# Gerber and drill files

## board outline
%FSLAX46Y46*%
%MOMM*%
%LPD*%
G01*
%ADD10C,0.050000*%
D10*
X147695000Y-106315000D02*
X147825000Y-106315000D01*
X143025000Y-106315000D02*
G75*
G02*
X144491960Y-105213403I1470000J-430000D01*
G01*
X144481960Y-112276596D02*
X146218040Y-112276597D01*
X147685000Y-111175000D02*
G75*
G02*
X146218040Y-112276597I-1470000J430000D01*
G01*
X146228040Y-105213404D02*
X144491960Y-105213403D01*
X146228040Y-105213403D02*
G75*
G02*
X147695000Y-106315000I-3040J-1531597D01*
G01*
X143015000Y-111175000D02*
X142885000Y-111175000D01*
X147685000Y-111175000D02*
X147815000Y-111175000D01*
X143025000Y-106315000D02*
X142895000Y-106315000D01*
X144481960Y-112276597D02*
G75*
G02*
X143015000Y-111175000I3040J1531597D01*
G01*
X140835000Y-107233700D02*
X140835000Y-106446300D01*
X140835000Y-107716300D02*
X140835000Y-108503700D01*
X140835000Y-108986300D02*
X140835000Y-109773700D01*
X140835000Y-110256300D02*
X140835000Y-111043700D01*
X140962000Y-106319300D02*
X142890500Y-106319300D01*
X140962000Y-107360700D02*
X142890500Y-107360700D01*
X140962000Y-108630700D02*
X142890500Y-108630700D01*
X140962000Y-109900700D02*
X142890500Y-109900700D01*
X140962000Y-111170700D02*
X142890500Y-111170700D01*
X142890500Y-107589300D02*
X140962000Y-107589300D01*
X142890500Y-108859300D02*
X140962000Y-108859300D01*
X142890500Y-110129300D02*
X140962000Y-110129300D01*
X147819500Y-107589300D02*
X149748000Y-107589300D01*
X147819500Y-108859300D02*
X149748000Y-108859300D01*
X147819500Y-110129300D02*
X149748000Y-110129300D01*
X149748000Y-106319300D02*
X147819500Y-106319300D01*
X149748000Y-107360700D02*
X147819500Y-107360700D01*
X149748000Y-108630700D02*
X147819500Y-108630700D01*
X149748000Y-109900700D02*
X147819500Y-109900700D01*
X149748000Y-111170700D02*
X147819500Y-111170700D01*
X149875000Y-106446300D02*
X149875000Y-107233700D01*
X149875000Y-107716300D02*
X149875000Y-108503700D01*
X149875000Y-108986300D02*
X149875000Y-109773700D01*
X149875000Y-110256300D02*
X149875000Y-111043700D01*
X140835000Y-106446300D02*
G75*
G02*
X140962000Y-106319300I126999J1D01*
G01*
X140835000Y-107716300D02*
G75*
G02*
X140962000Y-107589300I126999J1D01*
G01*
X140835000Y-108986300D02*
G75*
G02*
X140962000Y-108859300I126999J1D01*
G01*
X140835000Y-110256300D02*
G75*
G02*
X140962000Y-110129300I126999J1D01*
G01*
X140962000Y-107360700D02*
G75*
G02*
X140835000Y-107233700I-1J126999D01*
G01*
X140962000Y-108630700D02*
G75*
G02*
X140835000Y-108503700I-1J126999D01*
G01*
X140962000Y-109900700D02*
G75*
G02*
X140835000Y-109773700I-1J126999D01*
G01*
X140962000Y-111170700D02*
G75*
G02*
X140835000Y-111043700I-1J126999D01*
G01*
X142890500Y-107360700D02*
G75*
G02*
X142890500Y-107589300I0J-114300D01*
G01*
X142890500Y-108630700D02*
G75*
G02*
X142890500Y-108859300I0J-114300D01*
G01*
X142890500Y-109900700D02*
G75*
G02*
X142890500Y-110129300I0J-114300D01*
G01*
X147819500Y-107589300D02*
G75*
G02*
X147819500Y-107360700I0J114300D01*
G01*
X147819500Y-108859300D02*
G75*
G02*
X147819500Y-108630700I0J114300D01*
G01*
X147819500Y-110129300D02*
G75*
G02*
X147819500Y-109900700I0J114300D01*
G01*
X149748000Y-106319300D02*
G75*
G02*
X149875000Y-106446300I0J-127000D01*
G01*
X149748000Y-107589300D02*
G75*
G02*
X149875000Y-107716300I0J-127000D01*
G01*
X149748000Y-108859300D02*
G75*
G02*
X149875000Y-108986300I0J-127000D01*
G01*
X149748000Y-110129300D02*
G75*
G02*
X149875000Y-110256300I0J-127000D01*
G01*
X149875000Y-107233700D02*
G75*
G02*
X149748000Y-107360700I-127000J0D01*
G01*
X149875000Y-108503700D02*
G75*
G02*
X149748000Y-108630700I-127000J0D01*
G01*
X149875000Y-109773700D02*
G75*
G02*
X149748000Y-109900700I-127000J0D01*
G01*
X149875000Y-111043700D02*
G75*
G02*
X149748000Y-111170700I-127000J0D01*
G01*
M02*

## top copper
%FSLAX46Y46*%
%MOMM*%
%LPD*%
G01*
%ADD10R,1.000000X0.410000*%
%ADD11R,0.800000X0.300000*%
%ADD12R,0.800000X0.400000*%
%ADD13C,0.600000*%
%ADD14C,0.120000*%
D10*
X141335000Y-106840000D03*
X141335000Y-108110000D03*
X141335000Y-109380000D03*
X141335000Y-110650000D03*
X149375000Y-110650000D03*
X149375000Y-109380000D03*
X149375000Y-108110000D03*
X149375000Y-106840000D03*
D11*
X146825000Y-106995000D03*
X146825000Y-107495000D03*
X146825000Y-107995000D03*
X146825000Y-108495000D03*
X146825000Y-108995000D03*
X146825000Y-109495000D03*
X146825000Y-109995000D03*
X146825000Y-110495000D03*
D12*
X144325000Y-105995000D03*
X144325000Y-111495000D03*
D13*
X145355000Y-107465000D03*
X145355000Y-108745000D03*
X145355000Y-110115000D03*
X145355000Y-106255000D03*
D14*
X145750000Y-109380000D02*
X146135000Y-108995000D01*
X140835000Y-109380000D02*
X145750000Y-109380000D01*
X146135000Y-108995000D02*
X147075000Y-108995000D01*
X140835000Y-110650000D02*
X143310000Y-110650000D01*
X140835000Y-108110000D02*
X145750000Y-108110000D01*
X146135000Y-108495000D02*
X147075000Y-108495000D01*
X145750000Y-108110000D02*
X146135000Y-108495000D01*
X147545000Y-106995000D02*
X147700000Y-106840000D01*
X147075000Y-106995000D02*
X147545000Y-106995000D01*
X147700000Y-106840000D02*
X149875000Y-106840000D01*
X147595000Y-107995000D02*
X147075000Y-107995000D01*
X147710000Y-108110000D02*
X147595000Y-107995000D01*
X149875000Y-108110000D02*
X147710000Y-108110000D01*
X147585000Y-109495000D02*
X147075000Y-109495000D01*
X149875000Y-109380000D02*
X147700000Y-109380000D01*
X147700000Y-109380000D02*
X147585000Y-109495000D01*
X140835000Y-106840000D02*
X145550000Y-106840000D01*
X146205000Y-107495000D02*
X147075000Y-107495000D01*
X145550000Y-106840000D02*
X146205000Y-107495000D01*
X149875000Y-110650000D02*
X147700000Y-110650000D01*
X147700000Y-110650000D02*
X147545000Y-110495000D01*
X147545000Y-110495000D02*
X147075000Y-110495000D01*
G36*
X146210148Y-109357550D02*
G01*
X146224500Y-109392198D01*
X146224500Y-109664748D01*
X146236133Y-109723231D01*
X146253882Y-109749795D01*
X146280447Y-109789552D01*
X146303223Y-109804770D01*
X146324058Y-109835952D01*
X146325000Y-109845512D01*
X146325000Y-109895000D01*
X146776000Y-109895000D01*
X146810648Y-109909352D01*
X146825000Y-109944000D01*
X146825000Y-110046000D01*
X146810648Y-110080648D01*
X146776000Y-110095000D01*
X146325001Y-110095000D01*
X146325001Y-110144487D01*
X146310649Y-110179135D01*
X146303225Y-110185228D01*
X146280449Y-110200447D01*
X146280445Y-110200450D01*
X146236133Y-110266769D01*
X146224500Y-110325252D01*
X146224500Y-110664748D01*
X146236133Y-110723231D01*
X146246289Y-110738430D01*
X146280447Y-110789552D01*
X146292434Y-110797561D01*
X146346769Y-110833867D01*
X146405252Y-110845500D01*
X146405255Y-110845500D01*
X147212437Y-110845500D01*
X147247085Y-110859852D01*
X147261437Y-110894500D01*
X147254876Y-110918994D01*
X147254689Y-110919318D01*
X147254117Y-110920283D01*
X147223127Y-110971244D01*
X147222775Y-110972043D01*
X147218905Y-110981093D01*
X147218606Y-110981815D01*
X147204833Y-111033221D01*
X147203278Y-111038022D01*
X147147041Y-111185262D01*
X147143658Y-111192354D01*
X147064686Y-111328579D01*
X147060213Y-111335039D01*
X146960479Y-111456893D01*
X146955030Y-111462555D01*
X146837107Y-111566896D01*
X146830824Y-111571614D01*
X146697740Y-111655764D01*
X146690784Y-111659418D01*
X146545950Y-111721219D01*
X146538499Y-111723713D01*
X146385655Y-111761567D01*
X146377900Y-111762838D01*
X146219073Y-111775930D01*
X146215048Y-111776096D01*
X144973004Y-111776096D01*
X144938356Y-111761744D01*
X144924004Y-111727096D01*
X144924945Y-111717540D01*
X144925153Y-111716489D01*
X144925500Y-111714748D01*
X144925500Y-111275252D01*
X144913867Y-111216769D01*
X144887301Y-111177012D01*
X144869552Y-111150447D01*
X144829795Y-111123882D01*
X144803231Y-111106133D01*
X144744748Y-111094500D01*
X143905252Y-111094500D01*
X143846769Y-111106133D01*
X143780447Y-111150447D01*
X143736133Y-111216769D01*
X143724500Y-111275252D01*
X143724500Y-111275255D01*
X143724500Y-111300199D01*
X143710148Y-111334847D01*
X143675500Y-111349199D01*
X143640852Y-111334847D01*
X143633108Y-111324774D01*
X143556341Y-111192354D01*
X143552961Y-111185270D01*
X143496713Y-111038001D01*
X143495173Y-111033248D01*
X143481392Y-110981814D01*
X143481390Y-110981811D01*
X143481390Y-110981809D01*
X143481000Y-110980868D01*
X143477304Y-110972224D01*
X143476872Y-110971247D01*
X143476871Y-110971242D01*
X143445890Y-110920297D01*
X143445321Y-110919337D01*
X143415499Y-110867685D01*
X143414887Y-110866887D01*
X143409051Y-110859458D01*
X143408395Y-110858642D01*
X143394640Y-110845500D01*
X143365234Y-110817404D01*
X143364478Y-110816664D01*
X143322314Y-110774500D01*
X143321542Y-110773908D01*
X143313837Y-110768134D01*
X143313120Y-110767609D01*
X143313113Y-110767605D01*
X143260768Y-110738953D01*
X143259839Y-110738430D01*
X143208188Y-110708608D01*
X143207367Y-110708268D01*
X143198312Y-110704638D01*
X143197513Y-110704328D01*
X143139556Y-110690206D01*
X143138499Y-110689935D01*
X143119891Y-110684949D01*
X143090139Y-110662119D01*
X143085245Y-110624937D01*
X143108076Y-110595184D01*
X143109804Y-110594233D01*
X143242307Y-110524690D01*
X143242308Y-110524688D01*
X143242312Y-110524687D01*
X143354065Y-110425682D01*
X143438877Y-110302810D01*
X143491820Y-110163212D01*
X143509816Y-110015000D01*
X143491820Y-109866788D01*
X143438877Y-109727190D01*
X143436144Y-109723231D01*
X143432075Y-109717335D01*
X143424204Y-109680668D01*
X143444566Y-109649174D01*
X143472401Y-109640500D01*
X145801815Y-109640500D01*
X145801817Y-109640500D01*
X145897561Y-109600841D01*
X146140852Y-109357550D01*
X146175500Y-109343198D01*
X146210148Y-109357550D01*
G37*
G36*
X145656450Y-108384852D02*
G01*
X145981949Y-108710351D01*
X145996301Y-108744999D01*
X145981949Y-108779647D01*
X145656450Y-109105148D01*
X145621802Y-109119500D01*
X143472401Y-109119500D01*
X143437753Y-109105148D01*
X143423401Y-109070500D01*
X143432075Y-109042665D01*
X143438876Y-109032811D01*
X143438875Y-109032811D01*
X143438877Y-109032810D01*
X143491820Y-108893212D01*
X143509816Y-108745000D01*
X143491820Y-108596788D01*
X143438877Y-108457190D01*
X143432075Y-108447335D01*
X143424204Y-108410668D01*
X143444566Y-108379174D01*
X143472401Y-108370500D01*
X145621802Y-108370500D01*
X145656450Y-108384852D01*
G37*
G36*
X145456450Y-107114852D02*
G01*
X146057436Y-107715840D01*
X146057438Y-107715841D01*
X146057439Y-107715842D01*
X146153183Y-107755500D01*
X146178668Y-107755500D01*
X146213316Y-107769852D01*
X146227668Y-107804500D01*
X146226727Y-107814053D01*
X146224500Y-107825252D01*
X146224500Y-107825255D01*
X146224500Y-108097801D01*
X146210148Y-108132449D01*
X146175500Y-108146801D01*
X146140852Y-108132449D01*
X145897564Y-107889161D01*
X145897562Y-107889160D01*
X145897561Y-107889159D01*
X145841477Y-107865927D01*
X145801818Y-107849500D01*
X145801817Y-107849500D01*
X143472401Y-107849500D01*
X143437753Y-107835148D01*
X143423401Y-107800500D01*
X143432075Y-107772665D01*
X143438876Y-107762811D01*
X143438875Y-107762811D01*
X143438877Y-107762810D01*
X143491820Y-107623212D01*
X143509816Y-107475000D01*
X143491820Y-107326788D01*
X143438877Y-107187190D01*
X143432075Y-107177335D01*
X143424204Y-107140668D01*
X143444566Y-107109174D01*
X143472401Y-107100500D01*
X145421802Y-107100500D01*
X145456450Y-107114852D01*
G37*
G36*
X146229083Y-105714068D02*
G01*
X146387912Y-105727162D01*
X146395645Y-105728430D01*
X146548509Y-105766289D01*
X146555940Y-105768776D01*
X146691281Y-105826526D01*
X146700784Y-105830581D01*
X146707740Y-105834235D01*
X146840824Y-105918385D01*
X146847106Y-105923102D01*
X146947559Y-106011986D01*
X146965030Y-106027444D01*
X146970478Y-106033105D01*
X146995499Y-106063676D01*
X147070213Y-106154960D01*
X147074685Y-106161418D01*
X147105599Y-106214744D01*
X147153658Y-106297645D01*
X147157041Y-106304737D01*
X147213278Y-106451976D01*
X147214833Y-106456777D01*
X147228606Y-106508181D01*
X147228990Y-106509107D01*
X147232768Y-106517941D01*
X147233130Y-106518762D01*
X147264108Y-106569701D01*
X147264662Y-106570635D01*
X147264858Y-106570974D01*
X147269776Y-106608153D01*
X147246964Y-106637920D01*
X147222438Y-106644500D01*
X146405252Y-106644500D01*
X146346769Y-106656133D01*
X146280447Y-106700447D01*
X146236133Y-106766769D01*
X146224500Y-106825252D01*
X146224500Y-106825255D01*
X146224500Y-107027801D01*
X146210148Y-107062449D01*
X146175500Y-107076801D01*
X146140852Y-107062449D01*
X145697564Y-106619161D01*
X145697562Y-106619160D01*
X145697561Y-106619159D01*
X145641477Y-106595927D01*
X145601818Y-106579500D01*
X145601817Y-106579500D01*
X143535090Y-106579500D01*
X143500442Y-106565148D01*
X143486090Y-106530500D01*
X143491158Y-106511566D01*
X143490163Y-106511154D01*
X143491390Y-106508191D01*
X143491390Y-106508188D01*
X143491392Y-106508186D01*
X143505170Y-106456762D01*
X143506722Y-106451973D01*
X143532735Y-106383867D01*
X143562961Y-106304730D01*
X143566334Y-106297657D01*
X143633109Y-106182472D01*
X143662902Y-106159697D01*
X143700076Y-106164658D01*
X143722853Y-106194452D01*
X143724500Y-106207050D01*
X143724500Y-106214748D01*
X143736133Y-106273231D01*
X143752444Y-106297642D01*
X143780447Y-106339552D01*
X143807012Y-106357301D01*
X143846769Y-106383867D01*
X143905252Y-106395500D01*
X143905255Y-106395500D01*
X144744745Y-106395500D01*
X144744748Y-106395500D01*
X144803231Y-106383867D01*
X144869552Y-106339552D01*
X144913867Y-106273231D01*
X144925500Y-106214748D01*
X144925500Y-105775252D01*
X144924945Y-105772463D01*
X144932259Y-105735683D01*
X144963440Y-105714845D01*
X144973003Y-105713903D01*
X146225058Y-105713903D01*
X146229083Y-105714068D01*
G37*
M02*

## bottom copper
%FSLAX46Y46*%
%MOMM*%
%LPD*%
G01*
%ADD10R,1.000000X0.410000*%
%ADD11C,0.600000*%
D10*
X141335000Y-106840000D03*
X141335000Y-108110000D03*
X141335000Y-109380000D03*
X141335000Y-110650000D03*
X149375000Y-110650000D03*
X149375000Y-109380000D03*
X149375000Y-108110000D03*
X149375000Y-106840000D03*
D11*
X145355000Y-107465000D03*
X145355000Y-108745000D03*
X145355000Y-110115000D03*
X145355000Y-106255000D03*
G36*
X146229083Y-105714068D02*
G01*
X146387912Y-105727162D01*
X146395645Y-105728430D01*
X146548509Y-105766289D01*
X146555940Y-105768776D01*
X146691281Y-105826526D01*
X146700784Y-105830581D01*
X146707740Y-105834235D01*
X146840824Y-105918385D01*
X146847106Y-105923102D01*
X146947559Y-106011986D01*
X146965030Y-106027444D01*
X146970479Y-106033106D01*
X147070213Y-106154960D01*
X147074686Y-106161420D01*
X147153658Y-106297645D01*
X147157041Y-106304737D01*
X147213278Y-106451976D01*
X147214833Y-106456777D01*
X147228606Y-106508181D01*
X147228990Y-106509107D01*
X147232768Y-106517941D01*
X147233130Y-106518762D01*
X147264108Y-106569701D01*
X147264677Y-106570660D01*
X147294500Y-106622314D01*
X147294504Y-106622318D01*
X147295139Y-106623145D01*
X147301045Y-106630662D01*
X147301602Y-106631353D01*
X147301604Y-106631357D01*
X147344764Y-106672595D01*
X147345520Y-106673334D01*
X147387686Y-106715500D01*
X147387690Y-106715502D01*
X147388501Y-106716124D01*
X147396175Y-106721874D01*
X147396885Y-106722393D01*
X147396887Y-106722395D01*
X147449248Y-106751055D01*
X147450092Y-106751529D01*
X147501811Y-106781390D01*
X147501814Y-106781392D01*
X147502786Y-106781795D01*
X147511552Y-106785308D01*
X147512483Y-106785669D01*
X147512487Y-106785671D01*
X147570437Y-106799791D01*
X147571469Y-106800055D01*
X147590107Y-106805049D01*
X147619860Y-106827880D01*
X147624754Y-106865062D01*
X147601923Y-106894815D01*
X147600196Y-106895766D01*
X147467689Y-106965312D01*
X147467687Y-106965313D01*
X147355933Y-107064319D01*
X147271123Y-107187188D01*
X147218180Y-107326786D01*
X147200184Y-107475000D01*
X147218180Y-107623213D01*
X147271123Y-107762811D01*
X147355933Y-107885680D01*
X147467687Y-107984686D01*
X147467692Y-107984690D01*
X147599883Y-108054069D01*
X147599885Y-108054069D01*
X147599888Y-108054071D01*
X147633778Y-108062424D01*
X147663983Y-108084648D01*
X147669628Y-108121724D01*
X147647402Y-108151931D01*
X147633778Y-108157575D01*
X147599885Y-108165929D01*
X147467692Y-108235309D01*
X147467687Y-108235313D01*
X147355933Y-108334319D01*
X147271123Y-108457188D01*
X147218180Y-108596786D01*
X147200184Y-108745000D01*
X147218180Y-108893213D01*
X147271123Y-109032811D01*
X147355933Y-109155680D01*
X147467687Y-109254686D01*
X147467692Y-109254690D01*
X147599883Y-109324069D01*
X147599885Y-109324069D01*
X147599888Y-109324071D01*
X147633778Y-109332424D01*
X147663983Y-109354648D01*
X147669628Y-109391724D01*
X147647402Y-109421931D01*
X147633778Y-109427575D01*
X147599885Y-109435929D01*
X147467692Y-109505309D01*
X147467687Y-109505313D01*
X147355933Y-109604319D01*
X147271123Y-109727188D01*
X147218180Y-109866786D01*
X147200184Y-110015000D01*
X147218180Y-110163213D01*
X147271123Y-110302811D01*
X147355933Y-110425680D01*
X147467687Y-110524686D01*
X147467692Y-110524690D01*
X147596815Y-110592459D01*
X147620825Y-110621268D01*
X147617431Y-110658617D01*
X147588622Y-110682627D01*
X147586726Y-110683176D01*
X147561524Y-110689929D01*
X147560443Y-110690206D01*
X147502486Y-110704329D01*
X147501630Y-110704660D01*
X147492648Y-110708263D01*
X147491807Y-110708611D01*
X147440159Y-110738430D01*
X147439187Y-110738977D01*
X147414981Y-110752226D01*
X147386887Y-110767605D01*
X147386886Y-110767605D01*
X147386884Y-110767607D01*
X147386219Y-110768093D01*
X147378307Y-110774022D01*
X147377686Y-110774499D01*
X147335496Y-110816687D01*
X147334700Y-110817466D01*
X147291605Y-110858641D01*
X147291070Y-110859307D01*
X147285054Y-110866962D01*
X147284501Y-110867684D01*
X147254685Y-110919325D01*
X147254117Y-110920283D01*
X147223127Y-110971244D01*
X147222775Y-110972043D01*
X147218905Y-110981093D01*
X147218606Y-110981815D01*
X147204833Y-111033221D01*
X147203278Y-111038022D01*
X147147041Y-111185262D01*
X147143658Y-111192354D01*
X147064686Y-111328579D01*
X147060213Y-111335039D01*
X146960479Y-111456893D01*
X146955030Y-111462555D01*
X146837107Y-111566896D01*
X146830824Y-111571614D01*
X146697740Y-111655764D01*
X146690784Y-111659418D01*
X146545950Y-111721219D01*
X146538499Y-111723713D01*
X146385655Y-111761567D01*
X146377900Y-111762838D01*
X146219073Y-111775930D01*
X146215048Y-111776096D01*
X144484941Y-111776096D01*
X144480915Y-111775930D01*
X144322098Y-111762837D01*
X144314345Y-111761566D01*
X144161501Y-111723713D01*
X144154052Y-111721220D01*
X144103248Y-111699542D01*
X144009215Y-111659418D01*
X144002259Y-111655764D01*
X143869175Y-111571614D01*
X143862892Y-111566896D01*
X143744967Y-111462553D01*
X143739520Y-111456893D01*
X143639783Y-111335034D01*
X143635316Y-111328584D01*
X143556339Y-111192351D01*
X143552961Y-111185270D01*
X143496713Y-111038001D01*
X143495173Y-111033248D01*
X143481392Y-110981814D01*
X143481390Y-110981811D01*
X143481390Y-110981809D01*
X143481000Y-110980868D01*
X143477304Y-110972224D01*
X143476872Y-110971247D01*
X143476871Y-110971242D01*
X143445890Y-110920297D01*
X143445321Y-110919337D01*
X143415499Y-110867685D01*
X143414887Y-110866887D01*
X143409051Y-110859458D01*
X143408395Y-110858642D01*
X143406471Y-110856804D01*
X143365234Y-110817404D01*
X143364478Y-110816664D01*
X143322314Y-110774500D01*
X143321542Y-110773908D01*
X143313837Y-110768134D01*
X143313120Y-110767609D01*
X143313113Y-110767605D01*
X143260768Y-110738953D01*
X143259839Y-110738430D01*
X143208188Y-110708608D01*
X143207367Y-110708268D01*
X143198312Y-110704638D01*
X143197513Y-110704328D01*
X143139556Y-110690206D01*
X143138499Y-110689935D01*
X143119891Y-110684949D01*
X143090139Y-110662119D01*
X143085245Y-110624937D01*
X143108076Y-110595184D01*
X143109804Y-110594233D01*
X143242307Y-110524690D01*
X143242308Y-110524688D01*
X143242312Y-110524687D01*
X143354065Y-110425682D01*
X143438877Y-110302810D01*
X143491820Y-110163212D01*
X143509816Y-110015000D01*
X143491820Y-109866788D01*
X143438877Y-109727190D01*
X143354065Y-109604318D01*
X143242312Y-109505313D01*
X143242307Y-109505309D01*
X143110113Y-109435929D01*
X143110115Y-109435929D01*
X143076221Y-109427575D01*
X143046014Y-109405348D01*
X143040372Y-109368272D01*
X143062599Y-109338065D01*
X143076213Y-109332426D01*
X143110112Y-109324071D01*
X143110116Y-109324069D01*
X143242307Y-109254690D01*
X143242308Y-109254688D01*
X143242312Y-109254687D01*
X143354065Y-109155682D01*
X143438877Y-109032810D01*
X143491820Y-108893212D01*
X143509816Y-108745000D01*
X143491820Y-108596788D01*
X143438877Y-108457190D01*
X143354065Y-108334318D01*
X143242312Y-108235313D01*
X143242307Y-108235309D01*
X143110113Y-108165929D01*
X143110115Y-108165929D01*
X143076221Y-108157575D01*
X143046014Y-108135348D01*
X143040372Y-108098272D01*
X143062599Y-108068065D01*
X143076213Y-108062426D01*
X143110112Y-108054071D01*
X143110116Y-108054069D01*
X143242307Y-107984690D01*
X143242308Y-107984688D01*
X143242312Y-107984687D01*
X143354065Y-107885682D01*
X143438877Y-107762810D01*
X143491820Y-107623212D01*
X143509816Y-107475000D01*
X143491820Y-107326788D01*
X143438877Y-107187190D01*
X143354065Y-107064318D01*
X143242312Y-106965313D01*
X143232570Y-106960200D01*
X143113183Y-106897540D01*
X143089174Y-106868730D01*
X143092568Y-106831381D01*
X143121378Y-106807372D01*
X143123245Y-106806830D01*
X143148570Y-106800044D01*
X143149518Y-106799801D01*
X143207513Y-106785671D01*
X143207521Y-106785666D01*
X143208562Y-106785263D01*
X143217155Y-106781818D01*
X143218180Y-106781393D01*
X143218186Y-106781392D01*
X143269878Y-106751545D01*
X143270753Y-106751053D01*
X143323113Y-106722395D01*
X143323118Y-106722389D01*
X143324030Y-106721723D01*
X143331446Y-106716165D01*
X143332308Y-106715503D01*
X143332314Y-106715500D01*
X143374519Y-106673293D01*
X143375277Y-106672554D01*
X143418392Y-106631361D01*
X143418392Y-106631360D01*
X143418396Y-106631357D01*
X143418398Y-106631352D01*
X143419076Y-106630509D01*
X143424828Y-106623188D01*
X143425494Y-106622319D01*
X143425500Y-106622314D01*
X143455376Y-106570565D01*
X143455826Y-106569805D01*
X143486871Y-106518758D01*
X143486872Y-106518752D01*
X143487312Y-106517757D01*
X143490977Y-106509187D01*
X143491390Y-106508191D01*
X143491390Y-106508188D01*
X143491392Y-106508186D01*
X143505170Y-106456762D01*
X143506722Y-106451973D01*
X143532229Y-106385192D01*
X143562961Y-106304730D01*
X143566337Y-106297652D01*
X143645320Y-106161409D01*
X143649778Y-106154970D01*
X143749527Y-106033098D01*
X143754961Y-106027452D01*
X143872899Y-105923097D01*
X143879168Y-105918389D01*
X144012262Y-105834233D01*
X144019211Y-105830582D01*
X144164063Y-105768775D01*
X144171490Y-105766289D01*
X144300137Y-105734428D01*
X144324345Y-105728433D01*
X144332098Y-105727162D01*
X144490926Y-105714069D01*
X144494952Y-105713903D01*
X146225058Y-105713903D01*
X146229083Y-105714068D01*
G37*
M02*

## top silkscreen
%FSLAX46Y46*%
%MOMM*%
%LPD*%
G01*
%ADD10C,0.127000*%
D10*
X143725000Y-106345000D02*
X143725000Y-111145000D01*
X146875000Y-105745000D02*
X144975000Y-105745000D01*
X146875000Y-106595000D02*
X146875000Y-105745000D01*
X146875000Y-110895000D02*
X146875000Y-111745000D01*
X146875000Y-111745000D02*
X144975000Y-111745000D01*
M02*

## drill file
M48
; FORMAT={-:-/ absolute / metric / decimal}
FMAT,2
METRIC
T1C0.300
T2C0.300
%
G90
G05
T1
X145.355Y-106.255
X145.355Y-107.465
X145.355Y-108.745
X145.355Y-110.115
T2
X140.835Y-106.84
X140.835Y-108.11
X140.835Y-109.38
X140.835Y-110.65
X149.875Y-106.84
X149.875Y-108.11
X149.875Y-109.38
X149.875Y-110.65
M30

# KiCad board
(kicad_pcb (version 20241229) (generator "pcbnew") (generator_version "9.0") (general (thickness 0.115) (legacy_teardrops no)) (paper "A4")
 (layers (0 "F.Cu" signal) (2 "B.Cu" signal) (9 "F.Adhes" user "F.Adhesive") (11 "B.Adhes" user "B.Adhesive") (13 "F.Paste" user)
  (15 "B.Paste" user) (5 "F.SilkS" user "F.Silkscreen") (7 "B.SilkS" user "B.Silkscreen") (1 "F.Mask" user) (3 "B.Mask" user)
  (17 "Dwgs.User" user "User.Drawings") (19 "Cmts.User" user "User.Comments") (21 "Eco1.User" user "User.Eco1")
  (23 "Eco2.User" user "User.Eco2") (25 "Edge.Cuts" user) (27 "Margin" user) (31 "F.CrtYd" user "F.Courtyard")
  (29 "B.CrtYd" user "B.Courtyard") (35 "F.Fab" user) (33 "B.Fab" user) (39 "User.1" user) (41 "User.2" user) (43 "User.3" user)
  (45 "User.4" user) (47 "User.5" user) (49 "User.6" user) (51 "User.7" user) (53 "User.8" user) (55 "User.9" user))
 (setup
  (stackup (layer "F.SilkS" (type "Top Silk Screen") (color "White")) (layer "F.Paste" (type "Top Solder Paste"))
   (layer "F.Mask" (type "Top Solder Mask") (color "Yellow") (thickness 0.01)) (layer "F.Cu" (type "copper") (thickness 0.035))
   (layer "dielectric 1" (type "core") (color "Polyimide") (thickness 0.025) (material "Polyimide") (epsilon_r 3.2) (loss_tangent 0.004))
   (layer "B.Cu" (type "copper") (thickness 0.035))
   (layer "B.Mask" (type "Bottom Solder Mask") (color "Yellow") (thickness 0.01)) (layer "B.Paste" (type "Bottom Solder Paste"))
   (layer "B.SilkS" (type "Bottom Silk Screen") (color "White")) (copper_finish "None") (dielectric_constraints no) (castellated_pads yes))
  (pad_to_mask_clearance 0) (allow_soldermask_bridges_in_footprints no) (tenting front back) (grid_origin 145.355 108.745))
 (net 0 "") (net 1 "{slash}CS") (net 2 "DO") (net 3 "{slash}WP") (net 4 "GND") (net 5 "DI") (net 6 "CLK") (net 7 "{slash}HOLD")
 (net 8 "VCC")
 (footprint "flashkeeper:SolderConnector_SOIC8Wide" (layer "F.Cu") (at 145.355 108.745)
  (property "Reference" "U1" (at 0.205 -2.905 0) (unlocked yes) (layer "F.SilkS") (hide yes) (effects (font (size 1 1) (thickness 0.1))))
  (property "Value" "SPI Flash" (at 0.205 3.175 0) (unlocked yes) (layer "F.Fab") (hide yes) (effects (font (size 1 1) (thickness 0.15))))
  (fp_line (start -4.52 -1.5113) (end -4.52 -2.2987) (stroke (width 0.05) (type default)) (layer "Edge.Cuts"))
  (fp_line (start -4.52 -1.0287) (end -4.52 -0.2413) (stroke (width 0.05) (type default)) (layer "Edge.Cuts"))
  (fp_line (start -4.52 0.2413) (end -4.52 1.0287) (stroke (width 0.05) (type default)) (layer "Edge.Cuts"))
  (fp_line (start -4.52 1.5113) (end -4.52 2.2987) (stroke (width 0.05) (type default)) (layer "Edge.Cuts"))
  (fp_line (start -4.393 -2.4257) (end -2.4645 -2.4257) (stroke (width 0.05) (type default)) (layer "Edge.Cuts"))
  (fp_line (start -4.393 -1.3843) (end -2.4645 -1.3843) (stroke (width 0.05) (type default)) (layer "Edge.Cuts"))
  (fp_line (start -4.393 -0.1143) (end -2.4645 -0.1143) (stroke (width 0.05) (type default)) (layer "Edge.Cuts"))
  (fp_line (start -4.393 1.1557) (end -2.4645 1.1557) (stroke (width 0.05) (type default)) (layer "Edge.Cuts"))
  (fp_line (start -4.393 2.4257) (end -2.4645 2.4257) (stroke (width 0.05) (type default)) (layer "Edge.Cuts"))
  (fp_line (start -2.4645 -1.1557) (end -4.393 -1.1557) (stroke (width 0.05) (type default)) (layer "Edge.Cuts"))
  (fp_line (start -2.4645 0.1143) (end -4.393 0.1143) (stroke (width 0.05) (type default)) (layer "Edge.Cuts"))
  (fp_line (start -2.4645 1.3843) (end -4.393 1.3843) (stroke (width 0.05) (type default)) (layer "Edge.Cuts"))
  (fp_line (start 2.4645 -1.1557) (end 4.393 -1.1557) (stroke (width 0.05) (type default)) (layer "Edge.Cuts"))
  (fp_line (start 2.4645 0.1143) (end 4.393 0.1143) (stroke (width 0.05) (type default)) (layer "Edge.Cuts"))
  (fp_line (start 2.4645 1.3843) (end 4.393 1.3843) (stroke (width 0.05) (type default)) (layer "Edge.Cuts"))
  (fp_line (start 4.393 -2.4257) (end 2.4645 -2.4257) (stroke (width 0.05) (type default)) (layer "Edge.Cuts"))
  (fp_line (start 4.393 -1.3843) (end 2.4645 -1.3843) (stroke (width 0.05) (type default)) (layer "Edge.Cuts"))
  (fp_line (start 4.393 -0.1143) (end 2.4645 -0.1143) (stroke (width 0.05) (type default)) (layer "Edge.Cuts"))
  (fp_line (start 4.393 1.1557) (end 2.4645 1.1557) (stroke (width 0.05) (type default)) (layer "Edge.Cuts"))
  (fp_line (start 4.393 2.4257) (end 2.4645 2.4257) (stroke (width 0.05) (type default)) (layer "Edge.Cuts"))
  (fp_line (start 4.52 -2.2987) (end 4.52 -1.5113) (stroke (width 0.05) (type default)) (layer "Edge.Cuts"))
  (fp_line (start 4.52 -1.0287) (end 4.52 -0.2413) (stroke (width 0.05) (type default)) (layer "Edge.Cuts"))
  (fp_line (start 4.52 0.2413) (end 4.52 1.0287) (stroke (width 0.05) (type default)) (layer "Edge.Cuts"))
  (fp_line (start 4.52 1.5113) (end 4.52 2.2987) (stroke (width 0.05) (type default)) (layer "Edge.Cuts"))
  (fp_arc (start -4.52 -2.2987) (mid -4.482803 -2.388503) (end -4.393 -2.4257) (stroke (width 0.05) (type default)) (layer "Edge.Cuts"))
  (fp_arc (start -4.52 -1.0287) (mid -4.482803 -1.118503) (end -4.393 -1.1557) (stroke (width 0.05) (type default)) (layer "Edge.Cuts"))
  (fp_arc (start -4.52 0.2413) (mid -4.482803 0.151497) (end -4.393 0.1143) (stroke (width 0.05) (type default)) (layer "Edge.Cuts"))
  (fp_arc (start -4.52 1.5113) (mid -4.482803 1.421497) (end -4.393 1.3843) (stroke (width 0.05) (type default)) (layer "Edge.Cuts"))
  (fp_arc (start -4.393 -1.3843) (mid -4.482803 -1.421497) (end -4.52 -1.5113) (stroke (width 0.05) (type default)) (layer "Edge.Cuts"))
  (fp_arc (start -4.393 -0.1143) (mid -4.482803 -0.151497) (end -4.52 -0.2413) (stroke (width 0.05) (type default)) (layer "Edge.Cuts"))
  (fp_arc (start -4.393 1.1557) (mid -4.482803 1.118503) (end -4.52 1.0287) (stroke (width 0.05) (type default)) (layer "Edge.Cuts"))
  (fp_arc (start -4.393 2.4257) (mid -4.482803 2.388503) (end -4.52 2.2987) (stroke (width 0.05) (type default)) (layer "Edge.Cuts"))
  (fp_arc (start -2.4645 -1.3843) (mid -2.3502 -1.27) (end -2.4645 -1.1557) (stroke (width 0.05) (type default)) (layer "Edge.Cuts"))
  (fp_arc (start -2.4645 -0.1143) (mid -2.3502 0) (end -2.4645 0.1143) (stroke (width 0.05) (type default)) (layer "Edge.Cuts"))
  (fp_arc (start -2.4645 1.1557) (mid -2.3502 1.27) (end -2.4645 1.3843) (stroke (width 0.05) (type default)) (layer "Edge.Cuts"))
  (fp_arc (start 2.4645 -1.1557) (mid 2.3502 -1.27) (end 2.4645 -1.3843) (stroke (width 0.05) (type default)) (layer "Edge.Cuts"))
  (fp_arc (start 2.4645 0.1143) (mid 2.3502 0) (end 2.4645 -0.1143) (stroke (width 0.05) (type default)) (layer "Edge.Cuts"))
  (fp_arc (start 2.4645 1.3843) (mid 2.3502 1.27) (end 2.4645 1.1557) (stroke (width 0.05) (type default)) (layer "Edge.Cuts"))
  (fp_arc (start 4.393 -2.4257) (mid 4.482803 -2.388503) (end 4.52 -2.2987) (stroke (width 0.05) (type default)) (layer "Edge.Cuts"))
  (fp_arc (start 4.393 -1.1557) (mid 4.482803 -1.118503) (end 4.52 -1.0287) (stroke (width 0.05) (type default)) (layer "Edge.Cuts"))
  (fp_arc (start 4.393 0.1143) (mid 4.482803 0.151497) (end 4.52 0.2413) (stroke (width 0.05) (type default)) (layer "Edge.Cuts"))
  (fp_arc (start 4.393 1.3843) (mid 4.482803 1.421497) (end 4.52 1.5113) (stroke (width 0.05) (type default)) (layer "Edge.Cuts"))
  (fp_arc (start 4.52 -1.5113) (mid 4.482803 -1.421497) (end 4.393 -1.3843) (stroke (width 0.05) (type default)) (layer "Edge.Cuts"))
  (fp_arc (start 4.52 -0.2413) (mid 4.482803 -0.151497) (end 4.393 -0.1143) (stroke (width 0.05) (type default)) (layer "Edge.Cuts"))
  (fp_arc (start 4.52 1.0287) (mid 4.482803 1.118503) (end 4.393 1.1557) (stroke (width 0.05) (type default)) (layer "Edge.Cuts"))
  (fp_arc (start 4.52 2.2987) (mid 4.482803 2.388503) (end 4.393 2.4257) (stroke (width 0.05) (type default)) (layer "Edge.Cuts"))
  (pad "1" thru_hole rect (at -4.52 -1.905) (size 1 0.41) (drill 0.3 (offset 0.5 0)) (layers "*.Cu" "*.Mask") (remove_unused_layers no)
   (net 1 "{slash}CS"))
  (pad "2" thru_hole rect (at -4.52 -0.635) (size 1 0.41) (drill 0.3 (offset 0.5 0)) (layers "*.Cu" "*.Mask") (remove_unused_layers no)
   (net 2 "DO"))
  (pad "3" thru_hole rect (at -4.52 0.635) (size 1 0.41) (drill 0.3 (offset 0.5 0)) (layers "*.Cu" "*.Mask") (remove_unused_layers no)
   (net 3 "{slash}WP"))
  (pad "4" thru_hole rect (at -4.52 1.905) (size 1 0.41) (drill 0.3 (offset 0.5 0)) (layers "*.Cu" "*.Mask") (remove_unused_layers no)
   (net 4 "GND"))
  (pad "5" thru_hole rect (at 4.52 1.905 180) (size 1 0.41) (drill 0.3 (offset 0.5 0)) (layers "*.Cu" "*.Mask") (remove_unused_layers no)
   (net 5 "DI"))
  (pad "6" thru_hole rect (at 4.52 0.635 180) (size 1 0.41) (drill 0.3 (offset 0.5 0)) (layers "*.Cu" "*.Mask") (remove_unused_layers no)
   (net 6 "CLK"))
  (pad "7" thru_hole rect (at 4.52 -0.635 180) (size 1 0.41) (drill 0.3 (offset 0.5 0)) (layers "*.Cu" "*.Mask") (remove_unused_layers no)
   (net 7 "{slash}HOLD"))
  (pad "8" thru_hole rect (at 4.52 -1.905 180) (size 1 0.41) (drill 0.3 (offset 0.5 0)) (layers "*.Cu" "*.Mask") (remove_unused_layers no)
   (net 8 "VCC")))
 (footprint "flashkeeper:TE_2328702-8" (layer "F.Cu") (at 146.825 110.495 -90)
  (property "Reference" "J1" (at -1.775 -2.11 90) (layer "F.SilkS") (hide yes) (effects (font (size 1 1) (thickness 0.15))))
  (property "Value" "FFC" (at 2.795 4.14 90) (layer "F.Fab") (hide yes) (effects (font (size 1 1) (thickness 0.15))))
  (fp_line (start -4.15 3.1) (end 0.65 3.1) (stroke (width 0.127) (type solid)) (layer "F.SilkS"))
  (fp_line (start -4.75 -0.05) (end -4.75 1.85) (stroke (width 0.127) (type solid)) (layer "F.SilkS"))
  (fp_line (start -3.9 -0.05) (end -4.75 -0.05) (stroke (width 0.127) (type solid)) (layer "F.SilkS"))
  (fp_line (start 0.4 -0.05) (end 1.25 -0.05) (stroke (width 0.127) (type solid)) (layer "F.SilkS"))
  (fp_line (start 1.25 -0.05) (end 1.25 1.85) (stroke (width 0.127) (type solid)) (layer "F.SilkS"))
  (pad "1" smd rect (at -3.5 0 270) (size 0.3 0.8) (layers "F.Cu" "F.Mask" "F.Paste") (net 8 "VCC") (solder_mask_margin 0.102))
  (pad "2" smd rect (at -3 0 270) (size 0.3 0.8) (layers "F.Cu" "F.Mask" "F.Paste") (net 1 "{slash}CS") (solder_mask_margin 0.102))
  (pad "3" smd rect (at -2.5 0 270) (size 0.3 0.8) (layers "F.Cu" "F.Mask" "F.Paste") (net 7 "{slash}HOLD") (solder_mask_margin 0.102))
  (pad "4" smd rect (at -2 0 270) (size 0.3 0.8) (layers "F.Cu" "F.Mask" "F.Paste") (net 2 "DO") (solder_mask_margin 0.102))
  (pad "5" smd rect (at -1.5 0 270) (size 0.3 0.8) (layers "F.Cu" "F.Mask" "F.Paste") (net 3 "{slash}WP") (solder_mask_margin 0.102))
  (pad "6" smd rect (at -1 0 270) (size 0.3 0.8) (layers "F.Cu" "F.Mask" "F.Paste") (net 6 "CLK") (solder_mask_margin 0.102))
  (pad "7" smd rect (at -0.5 0 270) (size 0.3 0.8) (layers "F.Cu" "F.Mask" "F.Paste") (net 4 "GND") (solder_mask_margin 0.102))
  (pad "8" smd rect (at 0 0 270) (size 0.3 0.8) (layers "F.Cu" "F.Mask" "F.Paste") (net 5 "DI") (solder_mask_margin 0.102))
  (pad "S1" smd rect (at -4.5 2.5 270) (size 0.4 0.8) (layers "F.Cu" "F.Mask" "F.Paste") (solder_mask_margin 0.102))
  (pad "S2" smd rect (at 1 2.5 270) (size 0.4 0.8) (layers "F.Cu" "F.Mask" "F.Paste") (solder_mask_margin 0.102)))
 (gr_line (start 147.695 106.315) (end 147.825 106.315) (stroke (width 0.05) (type default)) (layer "Edge.Cuts"))
 (gr_arc (start 143.025 106.315) (mid 143.575304 105.520272) (end 144.49196 105.213403) (stroke (width 0.05) (type default))
  (layer "Edge.Cuts"))
 (gr_line (start 144.48196 112.276596) (end 146.21804 112.276597) (stroke (width 0.05) (type default)) (layer "Edge.Cuts"))
 (gr_arc (start 147.685 111.175) (mid 147.134696 111.969728) (end 146.21804 112.276597) (stroke (width 0.05) (type default))
  (layer "Edge.Cuts"))
 (gr_line (start 146.22804 105.213404) (end 144.49196 105.213403) (stroke (width 0.05) (type default)) (layer "Edge.Cuts"))
 (gr_arc (start 146.22804 105.213403) (mid 147.144696 105.520272) (end 147.695 106.315) (stroke (width 0.05) (type default))
  (layer "Edge.Cuts"))
 (gr_line (start 143.015 111.175) (end 142.885 111.175) (stroke (width 0.05) (type default)) (layer "Edge.Cuts"))
 (gr_line (start 147.685 111.175) (end 147.815 111.175) (stroke (width 0.05) (type default)) (layer "Edge.Cuts"))
 (gr_line (start 143.025 106.315) (end 142.895 106.315) (stroke (width 0.05) (type default)) (layer "Edge.Cuts"))
 (gr_arc (start 144.48196 112.276597) (mid 143.565304 111.969728) (end 143.015 111.175) (stroke (width 0.05) (type default))
  (layer "Edge.Cuts"))
 (segment (start 145.75 109.38) (end 146.135 108.995) (width 0.12) (layer "F.Cu") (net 3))
 (segment (start 140.835 109.38) (end 145.75 109.38) (width 0.12) (layer "F.Cu") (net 3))
 (segment (start 146.135 108.995) (end 147.075 108.995) (width 0.12) (layer "F.Cu") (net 3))
 (segment (start 140.835 110.65) (end 143.31 110.65) (width 0.12) (layer "F.Cu") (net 4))
 (via (at 145.355 107.465) (size 0.6) (drill 0.3) (layers "F.Cu" "B.Cu") (free yes) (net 4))
 (via (at 145.355 108.745) (size 0.6) (drill 0.3) (layers "F.Cu" "B.Cu") (free yes) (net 4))
 (via (at 145.355 110.115) (size 0.6) (drill 0.3) (layers "F.Cu" "B.Cu") (free yes) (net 4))
 (via (at 145.355 106.255) (size 0.6) (drill 0.3) (layers "F.Cu" "B.Cu") (free yes) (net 4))
 (segment (start 140.835 108.11) (end 145.75 108.11) (width 0.12) (layer "F.Cu") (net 2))
 (segment (start 146.135 108.495) (end 147.075 108.495) (width 0.12) (layer "F.Cu") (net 2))
 (segment (start 145.75 108.11) (end 146.135 108.495) (width 0.12) (layer "F.Cu") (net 2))
 (segment (start 147.545 106.995) (end 147.7 106.84) (width 0.12) (layer "F.Cu") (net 8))
 (segment (start 147.075 106.995) (end 147.545 106.995) (width 0.12) (layer "F.Cu") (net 8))
 (segment (start 147.7 106.84) (end 149.875 106.84) (width 0.12) (layer "F.Cu") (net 8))
 (segment (start 147.595 107.995) (end 147.075 107.995) (width 0.12) (layer "F.Cu") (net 7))
 (segment (start 147.71 108.11) (end 147.595 107.995) (width 0.12) (layer "F.Cu") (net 7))
 (segment (start 149.875 108.11) (end 147.71 108.11) (width 0.12) (layer "F.Cu") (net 7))
 (segment (start 147.585 109.495) (end 147.075 109.495) (width 0.12) (layer "F.Cu") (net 6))
 (segment (start 149.875 109.38) (end 147.7 109.38) (width 0.12) (layer "F.Cu") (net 6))
 (segment (start 147.7 109.38) (end 147.585 109.495) (width 0.12) (layer "F.Cu") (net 6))
 (segment (start 140.835 106.84) (end 145.55 106.84) (width 0.12) (layer "F.Cu") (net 1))
 (segment (start 146.205 107.495) (end 147.075 107.495) (width 0.12) (layer "F.Cu") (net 1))
 (segment (start 145.55 106.84) (end 146.205 107.495) (width 0.12) (layer "F.Cu") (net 1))
 (segment (start 149.875 110.65) (end 147.7 110.65) (width 0.12) (layer "F.Cu") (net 5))
 (segment (start 147.7 110.65) (end 147.545 110.495) (width 0.12) (layer "F.Cu") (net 5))
 (segment (start 147.545 110.495) (end 147.075 110.495) (width 0.12) (layer "F.Cu") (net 5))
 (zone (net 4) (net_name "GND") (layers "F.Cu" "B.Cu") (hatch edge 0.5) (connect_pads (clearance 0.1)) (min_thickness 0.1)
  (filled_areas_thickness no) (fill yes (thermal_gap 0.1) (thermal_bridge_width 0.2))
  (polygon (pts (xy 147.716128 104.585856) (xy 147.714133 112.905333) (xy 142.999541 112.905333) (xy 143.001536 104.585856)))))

